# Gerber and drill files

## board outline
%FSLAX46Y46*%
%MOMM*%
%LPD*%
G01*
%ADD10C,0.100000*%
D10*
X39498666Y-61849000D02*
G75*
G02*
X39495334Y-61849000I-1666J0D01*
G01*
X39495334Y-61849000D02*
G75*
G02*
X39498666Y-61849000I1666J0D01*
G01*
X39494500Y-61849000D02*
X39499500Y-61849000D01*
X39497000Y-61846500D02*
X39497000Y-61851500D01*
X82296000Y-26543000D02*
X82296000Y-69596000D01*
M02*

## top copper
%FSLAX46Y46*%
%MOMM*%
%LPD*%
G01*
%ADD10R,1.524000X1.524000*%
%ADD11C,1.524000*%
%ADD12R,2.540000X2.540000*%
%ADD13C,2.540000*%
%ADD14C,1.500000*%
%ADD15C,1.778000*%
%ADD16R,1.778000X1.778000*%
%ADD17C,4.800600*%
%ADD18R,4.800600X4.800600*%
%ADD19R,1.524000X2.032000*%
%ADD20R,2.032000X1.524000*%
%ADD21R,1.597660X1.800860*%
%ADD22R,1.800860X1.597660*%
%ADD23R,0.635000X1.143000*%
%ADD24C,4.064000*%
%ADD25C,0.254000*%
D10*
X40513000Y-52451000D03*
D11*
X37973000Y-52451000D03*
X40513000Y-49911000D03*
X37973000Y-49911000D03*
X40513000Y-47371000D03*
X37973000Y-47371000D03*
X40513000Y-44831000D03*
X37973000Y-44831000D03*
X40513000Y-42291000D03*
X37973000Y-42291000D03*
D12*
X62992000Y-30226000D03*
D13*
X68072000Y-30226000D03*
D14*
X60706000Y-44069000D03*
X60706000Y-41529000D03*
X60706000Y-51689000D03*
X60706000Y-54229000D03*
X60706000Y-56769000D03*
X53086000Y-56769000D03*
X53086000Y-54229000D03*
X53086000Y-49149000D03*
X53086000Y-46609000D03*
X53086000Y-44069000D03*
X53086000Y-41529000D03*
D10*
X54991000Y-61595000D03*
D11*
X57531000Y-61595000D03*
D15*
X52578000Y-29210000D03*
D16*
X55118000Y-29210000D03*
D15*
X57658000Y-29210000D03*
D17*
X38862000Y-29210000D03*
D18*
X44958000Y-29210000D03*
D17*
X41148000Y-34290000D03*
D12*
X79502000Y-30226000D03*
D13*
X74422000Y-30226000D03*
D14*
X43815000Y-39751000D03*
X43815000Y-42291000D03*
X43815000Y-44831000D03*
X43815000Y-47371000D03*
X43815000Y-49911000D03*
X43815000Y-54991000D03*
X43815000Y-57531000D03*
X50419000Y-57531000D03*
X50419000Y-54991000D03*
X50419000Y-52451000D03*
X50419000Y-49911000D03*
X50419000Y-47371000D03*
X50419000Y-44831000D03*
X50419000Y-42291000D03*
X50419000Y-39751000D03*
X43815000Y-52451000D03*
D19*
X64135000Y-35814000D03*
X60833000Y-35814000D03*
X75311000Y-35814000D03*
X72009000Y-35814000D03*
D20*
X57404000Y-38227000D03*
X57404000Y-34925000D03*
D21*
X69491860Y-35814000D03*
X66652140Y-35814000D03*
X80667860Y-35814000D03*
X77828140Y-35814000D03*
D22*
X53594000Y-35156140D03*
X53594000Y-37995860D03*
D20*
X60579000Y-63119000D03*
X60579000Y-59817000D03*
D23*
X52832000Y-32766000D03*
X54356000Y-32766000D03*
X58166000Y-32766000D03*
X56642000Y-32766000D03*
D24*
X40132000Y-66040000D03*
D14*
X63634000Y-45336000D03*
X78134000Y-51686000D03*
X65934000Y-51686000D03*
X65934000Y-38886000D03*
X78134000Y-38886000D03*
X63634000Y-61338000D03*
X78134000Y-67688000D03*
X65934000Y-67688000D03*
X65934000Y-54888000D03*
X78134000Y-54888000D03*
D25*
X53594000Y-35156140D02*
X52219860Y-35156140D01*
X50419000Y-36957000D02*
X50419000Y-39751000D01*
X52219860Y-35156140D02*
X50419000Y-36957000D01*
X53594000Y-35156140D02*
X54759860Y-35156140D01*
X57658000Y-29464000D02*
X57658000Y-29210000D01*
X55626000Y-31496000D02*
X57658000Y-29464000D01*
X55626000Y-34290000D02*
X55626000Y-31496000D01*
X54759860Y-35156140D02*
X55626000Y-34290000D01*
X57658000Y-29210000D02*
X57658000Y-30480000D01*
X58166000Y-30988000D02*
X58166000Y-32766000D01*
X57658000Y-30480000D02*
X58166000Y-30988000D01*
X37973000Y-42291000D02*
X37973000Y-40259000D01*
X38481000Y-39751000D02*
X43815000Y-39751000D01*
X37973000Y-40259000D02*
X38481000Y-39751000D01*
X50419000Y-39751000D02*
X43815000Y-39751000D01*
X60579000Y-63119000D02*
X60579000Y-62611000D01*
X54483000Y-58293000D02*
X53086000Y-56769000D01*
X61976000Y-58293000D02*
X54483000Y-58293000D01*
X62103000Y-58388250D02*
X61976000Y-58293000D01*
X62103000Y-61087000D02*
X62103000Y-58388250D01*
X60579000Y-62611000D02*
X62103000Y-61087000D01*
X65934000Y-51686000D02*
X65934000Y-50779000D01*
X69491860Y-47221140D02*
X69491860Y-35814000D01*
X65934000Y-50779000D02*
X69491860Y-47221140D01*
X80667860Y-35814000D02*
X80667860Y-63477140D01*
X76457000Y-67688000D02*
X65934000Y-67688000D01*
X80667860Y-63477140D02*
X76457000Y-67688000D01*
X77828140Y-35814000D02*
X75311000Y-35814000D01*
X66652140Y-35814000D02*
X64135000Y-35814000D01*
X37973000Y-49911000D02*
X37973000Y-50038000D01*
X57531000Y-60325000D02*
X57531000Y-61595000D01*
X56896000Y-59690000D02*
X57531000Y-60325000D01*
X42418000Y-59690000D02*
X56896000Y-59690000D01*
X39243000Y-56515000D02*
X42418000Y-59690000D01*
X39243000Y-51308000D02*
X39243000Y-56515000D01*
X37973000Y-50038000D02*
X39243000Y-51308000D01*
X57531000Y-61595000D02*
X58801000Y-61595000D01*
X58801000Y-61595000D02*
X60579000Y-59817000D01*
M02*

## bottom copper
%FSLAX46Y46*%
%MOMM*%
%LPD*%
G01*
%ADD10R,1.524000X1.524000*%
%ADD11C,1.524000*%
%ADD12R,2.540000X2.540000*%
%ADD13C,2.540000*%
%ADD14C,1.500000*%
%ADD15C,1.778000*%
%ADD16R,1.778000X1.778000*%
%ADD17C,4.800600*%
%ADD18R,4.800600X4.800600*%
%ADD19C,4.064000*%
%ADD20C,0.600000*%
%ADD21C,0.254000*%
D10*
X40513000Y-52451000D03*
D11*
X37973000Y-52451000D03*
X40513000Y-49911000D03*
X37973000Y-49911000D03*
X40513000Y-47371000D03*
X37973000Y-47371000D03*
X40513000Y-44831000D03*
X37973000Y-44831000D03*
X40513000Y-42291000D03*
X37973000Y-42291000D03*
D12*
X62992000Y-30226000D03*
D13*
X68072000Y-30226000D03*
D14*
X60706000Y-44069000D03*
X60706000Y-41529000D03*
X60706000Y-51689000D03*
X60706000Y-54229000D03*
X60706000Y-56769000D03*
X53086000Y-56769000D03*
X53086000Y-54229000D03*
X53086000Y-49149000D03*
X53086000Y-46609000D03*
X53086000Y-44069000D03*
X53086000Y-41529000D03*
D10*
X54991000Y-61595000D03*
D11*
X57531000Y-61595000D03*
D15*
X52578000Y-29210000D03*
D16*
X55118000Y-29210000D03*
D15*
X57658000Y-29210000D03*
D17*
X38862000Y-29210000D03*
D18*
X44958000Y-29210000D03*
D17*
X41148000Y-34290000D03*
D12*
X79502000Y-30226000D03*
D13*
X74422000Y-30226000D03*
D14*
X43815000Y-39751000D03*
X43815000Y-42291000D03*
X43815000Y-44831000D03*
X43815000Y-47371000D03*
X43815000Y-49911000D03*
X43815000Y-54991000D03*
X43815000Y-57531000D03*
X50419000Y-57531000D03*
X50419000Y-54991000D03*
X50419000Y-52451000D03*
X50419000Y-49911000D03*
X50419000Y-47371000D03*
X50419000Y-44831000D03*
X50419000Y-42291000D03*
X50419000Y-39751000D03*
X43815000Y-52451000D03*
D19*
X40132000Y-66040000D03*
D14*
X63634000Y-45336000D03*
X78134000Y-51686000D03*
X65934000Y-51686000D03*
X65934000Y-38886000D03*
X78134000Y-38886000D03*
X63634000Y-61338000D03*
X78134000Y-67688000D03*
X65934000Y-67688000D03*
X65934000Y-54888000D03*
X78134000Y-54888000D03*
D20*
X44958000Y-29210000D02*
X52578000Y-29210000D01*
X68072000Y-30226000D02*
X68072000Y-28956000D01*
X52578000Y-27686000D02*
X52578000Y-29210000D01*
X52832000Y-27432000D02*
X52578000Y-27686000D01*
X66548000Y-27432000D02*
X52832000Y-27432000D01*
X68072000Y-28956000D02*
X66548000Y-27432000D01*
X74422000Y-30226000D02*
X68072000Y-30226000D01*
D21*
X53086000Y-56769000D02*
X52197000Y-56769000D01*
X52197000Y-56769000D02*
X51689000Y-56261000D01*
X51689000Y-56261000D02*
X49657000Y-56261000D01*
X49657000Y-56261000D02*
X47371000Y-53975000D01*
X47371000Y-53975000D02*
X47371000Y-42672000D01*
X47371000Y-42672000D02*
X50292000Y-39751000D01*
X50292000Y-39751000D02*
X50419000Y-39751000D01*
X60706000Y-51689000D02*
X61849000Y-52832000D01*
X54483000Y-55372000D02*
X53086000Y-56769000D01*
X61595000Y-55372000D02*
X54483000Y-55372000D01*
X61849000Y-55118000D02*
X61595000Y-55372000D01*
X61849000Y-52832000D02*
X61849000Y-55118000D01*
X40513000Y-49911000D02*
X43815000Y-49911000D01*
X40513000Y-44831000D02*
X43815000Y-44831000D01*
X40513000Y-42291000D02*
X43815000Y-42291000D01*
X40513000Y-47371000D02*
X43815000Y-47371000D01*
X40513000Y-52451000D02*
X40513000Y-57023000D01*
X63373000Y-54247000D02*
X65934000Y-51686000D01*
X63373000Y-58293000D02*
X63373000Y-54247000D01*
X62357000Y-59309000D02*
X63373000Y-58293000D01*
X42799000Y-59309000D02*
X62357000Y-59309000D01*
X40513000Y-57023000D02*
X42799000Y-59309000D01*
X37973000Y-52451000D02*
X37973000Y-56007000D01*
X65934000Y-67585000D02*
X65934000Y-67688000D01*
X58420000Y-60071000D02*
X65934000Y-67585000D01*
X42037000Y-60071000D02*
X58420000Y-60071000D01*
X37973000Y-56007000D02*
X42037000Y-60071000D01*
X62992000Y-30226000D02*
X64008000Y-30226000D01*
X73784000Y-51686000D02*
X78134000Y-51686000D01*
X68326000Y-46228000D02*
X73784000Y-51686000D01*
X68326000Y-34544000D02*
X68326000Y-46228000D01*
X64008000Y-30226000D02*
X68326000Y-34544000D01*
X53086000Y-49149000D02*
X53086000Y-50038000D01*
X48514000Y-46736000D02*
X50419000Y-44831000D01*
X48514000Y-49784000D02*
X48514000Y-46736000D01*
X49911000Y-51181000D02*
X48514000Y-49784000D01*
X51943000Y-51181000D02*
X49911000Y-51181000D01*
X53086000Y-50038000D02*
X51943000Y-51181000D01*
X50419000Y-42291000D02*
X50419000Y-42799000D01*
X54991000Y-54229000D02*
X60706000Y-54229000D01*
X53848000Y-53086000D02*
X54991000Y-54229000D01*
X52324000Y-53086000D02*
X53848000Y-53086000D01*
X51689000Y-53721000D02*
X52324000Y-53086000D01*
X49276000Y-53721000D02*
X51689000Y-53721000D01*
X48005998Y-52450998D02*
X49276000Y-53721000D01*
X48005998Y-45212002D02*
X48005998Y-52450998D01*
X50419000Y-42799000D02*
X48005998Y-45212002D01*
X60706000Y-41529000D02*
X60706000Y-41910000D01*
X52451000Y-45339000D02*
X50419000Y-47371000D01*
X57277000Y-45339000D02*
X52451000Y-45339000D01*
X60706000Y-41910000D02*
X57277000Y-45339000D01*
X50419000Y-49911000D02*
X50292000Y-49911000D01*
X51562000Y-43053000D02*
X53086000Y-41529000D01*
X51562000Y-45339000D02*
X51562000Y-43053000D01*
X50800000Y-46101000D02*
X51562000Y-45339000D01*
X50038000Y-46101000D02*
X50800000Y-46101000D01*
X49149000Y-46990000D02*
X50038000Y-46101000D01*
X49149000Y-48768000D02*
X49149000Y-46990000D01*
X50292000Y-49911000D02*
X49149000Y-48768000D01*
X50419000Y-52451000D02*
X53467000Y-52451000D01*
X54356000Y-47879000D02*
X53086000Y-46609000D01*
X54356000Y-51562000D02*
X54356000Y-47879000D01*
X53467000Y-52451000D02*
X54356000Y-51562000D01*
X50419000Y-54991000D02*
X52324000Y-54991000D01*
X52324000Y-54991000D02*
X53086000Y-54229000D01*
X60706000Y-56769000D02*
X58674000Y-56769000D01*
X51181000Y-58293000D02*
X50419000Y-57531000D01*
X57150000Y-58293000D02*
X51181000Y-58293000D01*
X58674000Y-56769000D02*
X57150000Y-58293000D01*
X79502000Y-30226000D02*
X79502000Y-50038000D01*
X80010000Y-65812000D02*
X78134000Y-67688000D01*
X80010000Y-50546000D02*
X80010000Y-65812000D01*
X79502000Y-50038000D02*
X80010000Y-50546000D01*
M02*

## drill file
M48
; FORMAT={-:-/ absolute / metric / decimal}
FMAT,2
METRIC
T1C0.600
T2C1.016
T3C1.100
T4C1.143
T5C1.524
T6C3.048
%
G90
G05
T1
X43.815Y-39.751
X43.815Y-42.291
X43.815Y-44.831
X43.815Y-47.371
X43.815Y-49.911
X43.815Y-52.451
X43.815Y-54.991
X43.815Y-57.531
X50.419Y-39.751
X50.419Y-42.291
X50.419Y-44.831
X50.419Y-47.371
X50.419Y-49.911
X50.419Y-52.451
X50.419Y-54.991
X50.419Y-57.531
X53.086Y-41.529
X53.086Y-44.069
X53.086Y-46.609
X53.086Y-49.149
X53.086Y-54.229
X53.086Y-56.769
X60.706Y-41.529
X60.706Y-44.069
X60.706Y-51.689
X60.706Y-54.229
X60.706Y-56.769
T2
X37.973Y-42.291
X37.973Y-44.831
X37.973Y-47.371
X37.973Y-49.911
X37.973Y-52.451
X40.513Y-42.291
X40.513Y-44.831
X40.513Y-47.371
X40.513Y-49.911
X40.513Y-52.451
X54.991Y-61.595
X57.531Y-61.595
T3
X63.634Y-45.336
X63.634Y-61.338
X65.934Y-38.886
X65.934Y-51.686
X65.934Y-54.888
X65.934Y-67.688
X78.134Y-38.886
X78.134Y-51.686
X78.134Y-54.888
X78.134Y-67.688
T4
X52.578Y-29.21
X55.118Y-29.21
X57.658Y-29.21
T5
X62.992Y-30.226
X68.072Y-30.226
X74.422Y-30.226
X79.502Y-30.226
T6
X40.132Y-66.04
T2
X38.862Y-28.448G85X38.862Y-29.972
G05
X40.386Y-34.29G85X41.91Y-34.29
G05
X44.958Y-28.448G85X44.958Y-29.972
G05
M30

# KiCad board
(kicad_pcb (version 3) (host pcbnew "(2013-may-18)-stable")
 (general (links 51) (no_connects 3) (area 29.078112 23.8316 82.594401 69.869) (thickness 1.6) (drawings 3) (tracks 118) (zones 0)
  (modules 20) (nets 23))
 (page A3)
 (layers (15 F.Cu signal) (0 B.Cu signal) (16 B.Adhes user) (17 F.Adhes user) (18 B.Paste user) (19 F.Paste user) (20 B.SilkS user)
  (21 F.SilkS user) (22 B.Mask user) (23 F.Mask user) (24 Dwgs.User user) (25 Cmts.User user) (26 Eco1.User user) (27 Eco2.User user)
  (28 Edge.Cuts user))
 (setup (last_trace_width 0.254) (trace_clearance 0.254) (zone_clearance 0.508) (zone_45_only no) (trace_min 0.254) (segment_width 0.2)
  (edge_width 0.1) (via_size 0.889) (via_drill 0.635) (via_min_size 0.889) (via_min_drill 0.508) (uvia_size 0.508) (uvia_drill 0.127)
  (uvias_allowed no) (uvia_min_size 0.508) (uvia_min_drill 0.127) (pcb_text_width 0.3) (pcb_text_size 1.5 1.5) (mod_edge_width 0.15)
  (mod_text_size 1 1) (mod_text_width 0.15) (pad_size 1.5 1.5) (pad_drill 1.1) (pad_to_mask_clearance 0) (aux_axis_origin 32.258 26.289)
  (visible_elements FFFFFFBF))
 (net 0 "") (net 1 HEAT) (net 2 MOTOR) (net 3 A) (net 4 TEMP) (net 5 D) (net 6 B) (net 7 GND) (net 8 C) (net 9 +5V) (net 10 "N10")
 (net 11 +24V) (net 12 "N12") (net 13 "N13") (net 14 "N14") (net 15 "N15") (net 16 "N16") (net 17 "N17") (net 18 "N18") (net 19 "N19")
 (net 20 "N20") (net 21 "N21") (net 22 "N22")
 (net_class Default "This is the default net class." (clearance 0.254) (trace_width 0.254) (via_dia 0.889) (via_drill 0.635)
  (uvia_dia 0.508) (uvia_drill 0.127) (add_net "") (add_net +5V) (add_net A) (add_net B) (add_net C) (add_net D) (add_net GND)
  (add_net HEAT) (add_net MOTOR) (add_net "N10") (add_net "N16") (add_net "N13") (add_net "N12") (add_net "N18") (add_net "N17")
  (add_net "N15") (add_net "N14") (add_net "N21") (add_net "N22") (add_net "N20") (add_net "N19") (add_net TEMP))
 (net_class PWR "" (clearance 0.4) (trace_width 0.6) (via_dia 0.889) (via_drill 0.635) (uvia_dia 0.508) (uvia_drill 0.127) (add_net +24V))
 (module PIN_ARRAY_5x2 (layer F.Cu) (at 39.243 47.371 90)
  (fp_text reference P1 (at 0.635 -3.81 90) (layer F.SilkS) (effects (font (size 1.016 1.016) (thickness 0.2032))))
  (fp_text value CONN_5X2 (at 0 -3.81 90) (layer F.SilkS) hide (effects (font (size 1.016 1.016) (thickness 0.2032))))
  (pad 1 thru_hole rect (at -5.08 1.27 90) (size 1.524 1.524) (drill 1.016) (layers *.Cu *.Mask F.SilkS) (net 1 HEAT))
  (pad 2 thru_hole circle (at -5.08 -1.27 90) (size 1.524 1.524) (drill 1.016) (layers *.Cu *.Mask F.SilkS) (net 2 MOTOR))
  (pad 3 thru_hole circle (at -2.54 1.27 90) (size 1.524 1.524) (drill 1.016) (layers *.Cu *.Mask F.SilkS) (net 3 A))
  (pad 4 thru_hole circle (at -2.54 -1.27 90) (size 1.524 1.524) (drill 1.016) (layers *.Cu *.Mask F.SilkS) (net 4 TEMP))
  (pad 5 thru_hole circle (at 0 1.27 90) (size 1.524 1.524) (drill 1.016) (layers *.Cu *.Mask F.SilkS) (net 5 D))
  (pad 6 thru_hole circle (at 0 -1.27 90) (size 1.524 1.524) (drill 1.016) (layers *.Cu *.Mask F.SilkS))
  (pad 7 thru_hole circle (at 2.54 1.27 90) (size 1.524 1.524) (drill 1.016) (layers *.Cu *.Mask F.SilkS) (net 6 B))
  (pad 8 thru_hole circle (at 2.54 -1.27 90) (size 1.524 1.524) (drill 1.016) (layers *.Cu *.Mask F.SilkS) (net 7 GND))
  (pad 9 thru_hole circle (at 5.08 1.27 90) (size 1.524 1.524) (drill 1.016) (layers *.Cu *.Mask F.SilkS) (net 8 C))
  (pad 10 thru_hole circle (at 5.08 -1.27 90) (size 1.524 1.524) (drill 1.016) (layers *.Cu *.Mask F.SilkS) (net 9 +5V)))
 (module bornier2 (layer F.Cu) (at 65.532 30.226)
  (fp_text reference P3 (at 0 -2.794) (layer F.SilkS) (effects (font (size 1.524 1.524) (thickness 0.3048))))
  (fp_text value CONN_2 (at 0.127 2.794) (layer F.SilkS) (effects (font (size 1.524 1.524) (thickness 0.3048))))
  (pad 1 thru_hole rect (at -2.54 0) (size 2.54 2.54) (drill 1.524) (layers *.Cu *.Mask F.SilkS) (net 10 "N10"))
  (pad 2 thru_hole circle (at 2.54 0) (size 2.54 2.54) (drill 1.524) (layers *.Cu *.Mask F.SilkS) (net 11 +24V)))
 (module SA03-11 (layer F.Cu) (at 56.896 49.149 180)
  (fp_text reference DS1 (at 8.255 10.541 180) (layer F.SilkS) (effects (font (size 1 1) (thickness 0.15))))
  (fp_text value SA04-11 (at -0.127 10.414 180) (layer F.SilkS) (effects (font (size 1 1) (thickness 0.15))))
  (pad 6 thru_hole circle (at -3.81 5.08 180) (size 1.5 1.5) (drill 0.6) (layers *.Cu *.Mask F.SilkS))
  (pad 7 thru_hole circle (at -3.81 7.62 180) (size 1.5 1.5) (drill 0.6) (layers *.Cu *.Mask F.SilkS) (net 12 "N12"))
  (pad 3 thru_hole circle (at -3.81 -2.54 180) (size 1.5 1.5) (drill 0.6) (layers *.Cu *.Mask F.SilkS) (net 9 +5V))
  (pad 2 thru_hole circle (at -3.81 -5.08 180) (size 1.5 1.5) (drill 0.6) (layers *.Cu *.Mask F.SilkS) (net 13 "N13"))
  (pad 1 thru_hole circle (at -3.81 -7.62 180) (size 1.5 1.5) (drill 0.6) (layers *.Cu *.Mask F.SilkS) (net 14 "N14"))
  (pad 14 thru_hole circle (at 3.81 -7.62 180) (size 1.5 1.5) (drill 0.6) (layers *.Cu *.Mask F.SilkS) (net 9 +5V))
  (pad 13 thru_hole circle (at 3.81 -5.08 180) (size 1.5 1.5) (drill 0.6) (layers *.Cu *.Mask F.SilkS) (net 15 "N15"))
  (pad 11 thru_hole circle (at 3.81 0 180) (size 1.5 1.5) (drill 0.6) (layers *.Cu *.Mask F.SilkS) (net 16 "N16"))
  (pad 10 thru_hole circle (at 3.81 2.54 180) (size 1.5 1.5) (drill 0.6) (layers *.Cu *.Mask F.SilkS) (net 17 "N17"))
  (pad 9 thru_hole circle (at 3.81 5.08 180) (size 1.5 1.5) (drill 0.6) (layers *.Cu *.Mask F.SilkS))
  (pad 8 thru_hole circle (at 3.81 7.62 180) (size 1.5 1.5) (drill 0.6) (layers *.Cu *.Mask F.SilkS) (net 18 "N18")))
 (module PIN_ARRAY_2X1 (layer F.Cu) (at 56.261 61.595)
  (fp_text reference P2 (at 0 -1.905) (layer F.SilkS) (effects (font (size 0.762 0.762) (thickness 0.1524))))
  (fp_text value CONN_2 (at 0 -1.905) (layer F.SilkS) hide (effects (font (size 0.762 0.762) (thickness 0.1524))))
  (pad 1 thru_hole rect (at -1.27 0) (size 1.524 1.524) (drill 1.016) (layers *.Cu *.Mask F.SilkS) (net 7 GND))
  (pad 2 thru_hole circle (at 1.27 0) (size 1.524 1.524) (drill 1.016) (layers *.Cu *.Mask F.SilkS) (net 4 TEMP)))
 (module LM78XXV (layer F.Cu) (at 55.118 29.21 90)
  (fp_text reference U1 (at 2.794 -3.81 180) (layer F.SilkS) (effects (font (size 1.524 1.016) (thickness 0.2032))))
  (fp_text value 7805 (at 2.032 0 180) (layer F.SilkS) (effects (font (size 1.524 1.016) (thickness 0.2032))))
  (pad VI thru_hole circle (at 0 -2.54 90) (size 1.778 1.778) (drill 1.143) (layers *.Cu *.Mask F.SilkS) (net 11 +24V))
  (pad GND thru_hole rect (at 0 0 90) (size 1.778 1.778) (drill 1.143) (layers *.Cu *.Mask F.SilkS) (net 7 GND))
  (pad VO thru_hole circle (at 0 2.54 90) (size 1.778 1.778) (drill 1.143) (layers *.Cu *.Mask F.SilkS) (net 9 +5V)))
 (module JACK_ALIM (layer F.Cu) (at 38.862 29.21)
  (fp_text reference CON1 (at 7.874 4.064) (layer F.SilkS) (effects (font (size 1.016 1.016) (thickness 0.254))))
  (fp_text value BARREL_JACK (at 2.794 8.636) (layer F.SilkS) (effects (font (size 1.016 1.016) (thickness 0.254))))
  (pad 2 thru_hole circle (at 0 0) (size 4.8006 4.8006) (drill oval 1.016 2.54) (layers *.Cu *.Mask F.SilkS) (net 7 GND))
  (pad 1 thru_hole rect (at 6.096 0) (size 4.8006 4.8006) (drill oval 1.016 2.54) (layers *.Cu *.Mask F.SilkS) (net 11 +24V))
  (pad 3 thru_hole circle (at 2.286 5.08) (size 4.8006 4.8006) (drill oval 2.54 1.016) (layers *.Cu *.Mask F.SilkS) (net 7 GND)))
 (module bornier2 (layer F.Cu) (at 76.962 30.226 180)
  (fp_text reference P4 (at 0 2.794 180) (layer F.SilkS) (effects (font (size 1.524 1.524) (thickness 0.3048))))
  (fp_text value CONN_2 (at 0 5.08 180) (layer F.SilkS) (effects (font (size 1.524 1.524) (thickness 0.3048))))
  (pad 1 thru_hole rect (at -2.54 0 180) (size 2.54 2.54) (drill 1.524) (layers *.Cu *.Mask F.SilkS) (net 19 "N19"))
  (pad 2 thru_hole circle (at 2.54 0 180) (size 2.54 2.54) (drill 1.524) (layers *.Cu *.Mask F.SilkS) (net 11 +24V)))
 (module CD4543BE (layer F.Cu) (at 47.117 48.641 270)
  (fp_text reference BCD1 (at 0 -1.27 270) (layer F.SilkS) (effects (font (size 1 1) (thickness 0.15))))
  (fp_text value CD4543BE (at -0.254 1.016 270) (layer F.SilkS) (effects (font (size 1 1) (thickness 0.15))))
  (pad 1 thru_hole circle (at -8.89 3.302 270) (size 1.5 1.5) (drill 0.6) (layers *.Cu *.Mask F.SilkS) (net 9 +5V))
  (pad 2 thru_hole circle (at -6.35 3.302 270) (size 1.5 1.5) (drill 0.6) (layers *.Cu *.Mask F.SilkS) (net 8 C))
  (pad 3 thru_hole circle (at -3.81 3.302 270) (size 1.5 1.5) (drill 0.6) (layers *.Cu *.Mask F.SilkS) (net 6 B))
  (pad 4 thru_hole circle (at -1.27 3.302 270) (size 1.5 1.5) (drill 0.6) (layers *.Cu *.Mask F.SilkS) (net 5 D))
  (pad 5 thru_hole circle (at 1.27 3.302 270) (size 1.5 1.5) (drill 0.6) (layers *.Cu *.Mask F.SilkS) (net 3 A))
  (pad 7 thru_hole circle (at 6.35 3.302 270) (size 1.5 1.5) (drill 0.6) (layers *.Cu *.Mask F.SilkS) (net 7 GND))
  (pad 8 thru_hole circle (at 8.89 3.302 270) (size 1.5 1.5) (drill 0.6) (layers *.Cu *.Mask F.SilkS) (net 7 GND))
  (pad 9 thru_hole circle (at 8.89 -3.302 270) (size 1.5 1.5) (drill 0.6) (layers *.Cu *.Mask F.SilkS) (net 14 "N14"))
  (pad 10 thru_hole circle (at 6.35 -3.302 270) (size 1.5 1.5) (drill 0.6) (layers *.Cu *.Mask F.SilkS) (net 15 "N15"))
  (pad 11 thru_hole circle (at 3.81 -3.302 270) (size 1.5 1.5) (drill 0.6) (layers *.Cu *.Mask F.SilkS) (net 17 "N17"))
  (pad 12 thru_hole circle (at 1.27 -3.302 270) (size 1.5 1.5) (drill 0.6) (layers *.Cu *.Mask F.SilkS) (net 18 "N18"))
  (pad 13 thru_hole circle (at -1.27 -3.302 270) (size 1.5 1.5) (drill 0.6) (layers *.Cu *.Mask F.SilkS) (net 12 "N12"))
  (pad 14 thru_hole circle (at -3.81 -3.302 270) (size 1.5 1.5) (drill 0.6) (layers *.Cu *.Mask F.SilkS) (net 16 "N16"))
  (pad 15 thru_hole circle (at -6.35 -3.302 270) (size 1.5 1.5) (drill 0.6) (layers *.Cu *.Mask F.SilkS) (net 13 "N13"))
  (pad 16 thru_hole circle (at -8.89 -3.302 270) (size 1.5 1.5) (drill 0.6) (layers *.Cu *.Mask F.SilkS) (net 9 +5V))
  (pad 6 thru_hole circle (at 3.81 3.302 270) (size 1.5 1.5) (drill 0.6) (layers *.Cu *.Mask F.SilkS)))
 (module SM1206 (layer F.Cu) (at 62.484 35.814 180)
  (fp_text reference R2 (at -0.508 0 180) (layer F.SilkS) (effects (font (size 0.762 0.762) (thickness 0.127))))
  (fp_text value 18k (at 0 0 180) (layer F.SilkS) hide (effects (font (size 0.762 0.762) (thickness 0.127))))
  (pad 1 smd rect (at -1.651 0 180) (size 1.524 2.032) (layers F.Cu F.Paste F.Mask) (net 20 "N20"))
  (pad 2 smd rect (at 1.651 0 180) (size 1.524 2.032) (layers F.Cu F.Paste F.Mask) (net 7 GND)))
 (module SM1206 (layer F.Cu) (at 73.66 35.814 180)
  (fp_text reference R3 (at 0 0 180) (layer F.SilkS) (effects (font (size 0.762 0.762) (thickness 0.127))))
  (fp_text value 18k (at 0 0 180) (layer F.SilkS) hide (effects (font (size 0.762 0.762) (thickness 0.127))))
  (pad 1 smd rect (at -1.651 0 180) (size 1.524 2.032) (layers F.Cu F.Paste F.Mask) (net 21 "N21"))
  (pad 2 smd rect (at 1.651 0 180) (size 1.524 2.032) (layers F.Cu F.Paste F.Mask) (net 7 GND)))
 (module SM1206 (layer F.Cu) (at 57.404 36.576 90)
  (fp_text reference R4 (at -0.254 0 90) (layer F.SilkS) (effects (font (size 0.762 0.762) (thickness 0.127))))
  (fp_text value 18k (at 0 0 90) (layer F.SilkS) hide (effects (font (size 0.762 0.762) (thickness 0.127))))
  (pad 1 smd rect (at -1.651 0 90) (size 1.524 2.032) (layers F.Cu F.Paste F.Mask) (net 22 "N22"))
  (pad 2 smd rect (at 1.651 0 90) (size 1.524 2.032) (layers F.Cu F.Paste F.Mask) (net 7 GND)))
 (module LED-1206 (layer F.Cu) (at 68.072 35.814 180)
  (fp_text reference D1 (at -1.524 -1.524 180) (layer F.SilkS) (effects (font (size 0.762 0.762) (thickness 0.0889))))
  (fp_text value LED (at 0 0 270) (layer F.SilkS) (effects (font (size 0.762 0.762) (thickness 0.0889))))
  (pad 1 smd rect (at -1.41986 0 180) (size 1.59766 1.80086) (layers F.Cu F.Paste F.Mask) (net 1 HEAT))
  (pad 2 smd rect (at 1.41986 0 180) (size 1.59766 1.80086) (layers F.Cu F.Paste F.Mask) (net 20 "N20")))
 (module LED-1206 (layer F.Cu) (at 79.248 35.814 180)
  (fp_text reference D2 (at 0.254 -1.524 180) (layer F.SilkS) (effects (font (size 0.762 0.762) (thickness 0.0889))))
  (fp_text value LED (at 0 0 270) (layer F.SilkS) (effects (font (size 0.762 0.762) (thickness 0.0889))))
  (pad 1 smd rect (at -1.41986 0 180) (size 1.59766 1.80086) (layers F.Cu F.Paste F.Mask) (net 2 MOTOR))
  (pad 2 smd rect (at 1.41986 0 180) (size 1.59766 1.80086) (layers F.Cu F.Paste F.Mask) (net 21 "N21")))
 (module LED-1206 (layer F.Cu) (at 53.594 36.576 270)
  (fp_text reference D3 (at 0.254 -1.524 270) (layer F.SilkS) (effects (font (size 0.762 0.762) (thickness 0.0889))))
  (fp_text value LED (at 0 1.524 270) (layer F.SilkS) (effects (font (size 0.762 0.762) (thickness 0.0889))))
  (pad 1 smd rect (at -1.41986 0 270) (size 1.59766 1.80086) (layers F.Cu F.Paste F.Mask) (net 9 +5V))
  (pad 2 smd rect (at 1.41986 0 270) (size 1.59766 1.80086) (layers F.Cu F.Paste F.Mask) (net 22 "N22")))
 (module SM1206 (layer F.Cu) (at 60.579 61.468 90)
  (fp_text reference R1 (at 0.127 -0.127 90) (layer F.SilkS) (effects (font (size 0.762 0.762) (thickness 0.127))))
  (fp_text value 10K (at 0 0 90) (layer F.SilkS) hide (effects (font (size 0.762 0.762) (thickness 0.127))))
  (pad 1 smd rect (at -1.651 0 90) (size 1.524 2.032) (layers F.Cu F.Paste F.Mask) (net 9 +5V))
  (pad 2 smd rect (at 1.651 0 90) (size 1.524 2.032) (layers F.Cu F.Paste F.Mask) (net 4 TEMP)))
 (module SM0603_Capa (layer F.Cu) (at 53.594 32.766)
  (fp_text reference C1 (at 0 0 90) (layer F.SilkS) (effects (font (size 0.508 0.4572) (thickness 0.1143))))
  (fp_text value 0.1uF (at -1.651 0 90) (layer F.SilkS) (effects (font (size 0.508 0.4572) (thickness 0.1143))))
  (pad 1 smd rect (at -0.762 0) (size 0.635 1.143) (layers F.Cu F.Paste F.Mask) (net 11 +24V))
  (pad 2 smd rect (at 0.762 0) (size 0.635 1.143) (layers F.Cu F.Paste F.Mask) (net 7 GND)))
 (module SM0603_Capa (layer F.Cu) (at 57.404 32.766 180)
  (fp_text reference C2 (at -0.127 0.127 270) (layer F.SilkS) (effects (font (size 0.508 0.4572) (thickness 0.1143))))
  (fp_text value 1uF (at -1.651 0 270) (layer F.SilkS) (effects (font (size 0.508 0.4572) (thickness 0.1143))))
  (pad 1 smd rect (at -0.762 0 180) (size 0.635 1.143) (layers F.Cu F.Paste F.Mask) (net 9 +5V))
  (pad 2 smd rect (at 0.762 0 180) (size 0.635 1.143) (layers F.Cu F.Paste F.Mask) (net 7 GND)))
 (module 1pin (layer F.Cu) (at 40.132 66.04)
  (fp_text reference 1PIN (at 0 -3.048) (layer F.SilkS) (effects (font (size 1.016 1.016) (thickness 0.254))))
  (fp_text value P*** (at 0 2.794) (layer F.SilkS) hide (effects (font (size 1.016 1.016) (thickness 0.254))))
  (pad 1 thru_hole circle (at 0 0) (size 4.064 4.064) (drill 3.048) (layers *.Cu *.Mask F.SilkS)))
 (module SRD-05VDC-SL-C (layer F.Cu) (at 81.534 53.086 180)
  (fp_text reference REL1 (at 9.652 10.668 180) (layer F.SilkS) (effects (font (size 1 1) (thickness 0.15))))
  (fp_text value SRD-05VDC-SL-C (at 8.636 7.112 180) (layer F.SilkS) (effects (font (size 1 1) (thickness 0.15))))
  (pad 5 thru_hole circle (at 17.9 7.75 180) (size 1.5 1.5) (drill 1.1) (layers *.Cu *.Mask F.SilkS) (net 7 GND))
  (pad 2 thru_hole circle (at 3.4 1.4 180) (size 1.5 1.5) (drill 1.1) (layers *.Cu *.Mask F.SilkS) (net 10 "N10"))
  (pad 1 thru_hole circle (at 15.6 1.4 180) (size 1.5 1.5) (drill 1.1) (layers *.Cu *.Mask F.SilkS) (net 1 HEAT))
  (pad 4 thru_hole circle (at 15.6 14.2 180) (size 1.5 1.5) (drill 1.1) (layers *.Cu *.Mask F.SilkS) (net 7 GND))
  (pad 3 thru_hole circle (at 3.4 14.2 180) (size 1.5 1.5) (drill 1.1) (layers *.Cu *.Mask F.SilkS) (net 7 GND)))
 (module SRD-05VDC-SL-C (layer F.Cu) (at 81.534 69.088 180)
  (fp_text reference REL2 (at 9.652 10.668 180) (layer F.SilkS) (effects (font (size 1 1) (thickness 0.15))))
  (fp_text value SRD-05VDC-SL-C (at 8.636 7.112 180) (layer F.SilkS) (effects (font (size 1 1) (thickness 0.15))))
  (pad 5 thru_hole circle (at 17.9 7.75 180) (size 1.5 1.5) (drill 1.1) (layers *.Cu *.Mask F.SilkS) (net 7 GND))
  (pad 2 thru_hole circle (at 3.4 1.4 180) (size 1.5 1.5) (drill 1.1) (layers *.Cu *.Mask F.SilkS) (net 19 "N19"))
  (pad 1 thru_hole circle (at 15.6 1.4 180) (size 1.5 1.5) (drill 1.1) (layers *.Cu *.Mask F.SilkS) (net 2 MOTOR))
  (pad 4 thru_hole circle (at 15.6 14.2 180) (size 1.5 1.5) (drill 1.1) (layers *.Cu *.Mask F.SilkS) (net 7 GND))
  (pad 3 thru_hole circle (at 3.4 14.2 180) (size 1.5 1.5) (drill 1.1) (layers *.Cu *.Mask F.SilkS) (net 7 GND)))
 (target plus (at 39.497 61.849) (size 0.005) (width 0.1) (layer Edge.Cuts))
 (gr_line (start 82.296 26.543) (end 82.296 69.596) (angle 90) (layer Edge.Cuts) (width 0.1))
 (segment (start 44.958 29.21) (end 52.578 29.21) (width 0.6) (layer B.Cu) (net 11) (status C00000))
 (segment (start 68.072 30.226) (end 68.072 28.956) (width 0.6) (layer B.Cu) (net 11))
 (segment (start 52.578 27.686) (end 52.578 29.21) (width 0.6) (layer B.Cu) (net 11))
 (segment (start 52.832 27.432) (end 52.578 27.686) (width 0.6) (layer B.Cu) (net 11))
 (segment (start 66.548 27.432) (end 52.832 27.432) (width 0.6) (layer B.Cu) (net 11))
 (segment (start 68.072 28.956) (end 66.548 27.432) (width 0.6) (layer B.Cu) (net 11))
 (segment (start 74.422 30.226) (end 68.072 30.226) (width 0.6) (layer B.Cu) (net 11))
 (segment (start 53.594 35.15614) (end 52.21986 35.15614) (width 0.254) (layer F.Cu) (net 9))
 (segment (start 50.419 36.957) (end 50.419 39.751) (width 0.254) (layer F.Cu) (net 9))
 (segment (start 52.21986 35.15614) (end 50.419 36.957) (width 0.254) (layer F.Cu) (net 9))
 (segment (start 53.594 35.15614) (end 54.75986 35.15614) (width 0.254) (layer F.Cu) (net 9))
 (segment (start 57.658 29.464) (end 57.658 29.21) (width 0.254) (layer F.Cu) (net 9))
 (segment (start 55.626 31.496) (end 57.658 29.464) (width 0.254) (layer F.Cu) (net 9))
 (segment (start 55.626 34.29) (end 55.626 31.496) (width 0.254) (layer F.Cu) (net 9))
 (segment (start 54.75986 35.15614) (end 55.626 34.29) (width 0.254) (layer F.Cu) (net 9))
 (segment (start 57.658 29.21) (end 57.658 30.48) (width 0.254) (layer F.Cu) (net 9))
 (segment (start 58.166 30.988) (end 58.166 32.766) (width 0.254) (layer F.Cu) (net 9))
 (segment (start 57.658 30.48) (end 58.166 30.988) (width 0.254) (layer F.Cu) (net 9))
 (segment (start 37.973 42.291) (end 37.973 40.259) (width 0.254) (layer F.Cu) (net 9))
 (segment (start 38.481 39.751) (end 43.815 39.751) (width 0.254) (layer F.Cu) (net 9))
 (segment (start 37.973 40.259) (end 38.481 39.751) (width 0.254) (layer F.Cu) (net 9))
 (segment (start 50.419 39.751) (end 43.815 39.751) (width 0.254) (layer F.Cu) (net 9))
 (segment (start 60.579 63.119) (end 60.579 62.611) (width 0.254) (layer F.Cu) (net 9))
 (segment (start 54.483 58.293) (end 53.086 56.769) (width 0.254) (layer F.Cu) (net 9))
 (segment (start 61.976 58.293) (end 54.483 58.293) (width 0.254) (layer F.Cu) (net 9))
 (segment (start 62.103 58.38825) (end 61.976 58.293) (width 0.254) (layer F.Cu) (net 9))
 (segment (start 62.103 61.087) (end 62.103 58.38825) (width 0.254) (layer F.Cu) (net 9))
 (segment (start 60.579 62.611) (end 62.103 61.087) (width 0.254) (layer F.Cu) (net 9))
 (segment (start 53.086 56.769) (end 52.197 56.769) (width 0.254) (layer B.Cu) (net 9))
 (segment (start 52.197 56.769) (end 51.689 56.261) (width 0.254) (layer B.Cu) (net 9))
 (segment (start 51.689 56.261) (end 49.657 56.261) (width 0.254) (layer B.Cu) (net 9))
 (segment (start 49.657 56.261) (end 47.371 53.975) (width 0.254) (layer B.Cu) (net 9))
 (segment (start 47.371 53.975) (end 47.371 42.672) (width 0.254) (layer B.Cu) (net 9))
 (segment (start 47.371 42.672) (end 50.292 39.751) (width 0.254) (layer B.Cu) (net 9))
 (segment (start 50.292 39.751) (end 50.419 39.751) (width 0.254) (layer B.Cu) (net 9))
 (segment (start 60.706 51.689) (end 61.849 52.832) (width 0.254) (layer B.Cu) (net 9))
 (segment (start 54.483 55.372) (end 53.086 56.769) (width 0.254) (layer B.Cu) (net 9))
 (segment (start 61.595 55.372) (end 54.483 55.372) (width 0.254) (layer B.Cu) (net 9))
 (segment (start 61.849 55.118) (end 61.595 55.372) (width 0.254) (layer B.Cu) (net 9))
 (segment (start 61.849 52.832) (end 61.849 55.118) (width 0.254) (layer B.Cu) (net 9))
 (segment (start 40.513 49.911) (end 43.815 49.911) (width 0.254) (layer B.Cu) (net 3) (status 10))
 (segment (start 40.513 44.831) (end 43.815 44.831) (width 0.254) (layer B.Cu) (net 6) (status 10))
 (segment (start 40.513 42.291) (end 43.815 42.291) (width 0.254) (layer B.Cu) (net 8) (status 10))
 (segment (start 40.513 47.371) (end 43.815 47.371) (width 0.254) (layer B.Cu) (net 5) (status 10))
 (segment (start 40.513 52.451) (end 40.513 57.023) (width 0.254) (layer B.Cu) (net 1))
 (segment (start 63.373 54.247) (end 65.934 51.686) (width 0.254) (layer B.Cu) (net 1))
 (segment (start 63.373 58.293) (end 63.373 54.247) (width 0.254) (layer B.Cu) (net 1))
 (segment (start 62.357 59.309) (end 63.373 58.293) (width 0.254) (layer B.Cu) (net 1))
 (segment (start 42.799 59.309) (end 62.357 59.309) (width 0.254) (layer B.Cu) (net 1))
 (segment (start 40.513 57.023) (end 42.799 59.309) (width 0.254) (layer B.Cu) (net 1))
 (segment (start 65.934 51.686) (end 65.934 50.779) (width 0.254) (layer F.Cu) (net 1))
 (segment (start 69.49186 47.22114) (end 69.49186 35.814) (width 0.254) (layer F.Cu) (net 1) (status 20))
 (segment (start 65.934 50.779) (end 69.49186 47.22114) (width 0.254) (layer F.Cu) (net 1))
 (segment (start 37.973 52.451) (end 37.973 56.007) (width 0.254) (layer B.Cu) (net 2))
 (segment (start 65.934 67.585) (end 65.934 67.688) (width 0.254) (layer B.Cu) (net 2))
 (segment (start 58.42 60.071) (end 65.934 67.585) (width 0.254) (layer B.Cu) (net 2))
 (segment (start 42.037 60.071) (end 58.42 60.071) (width 0.254) (layer B.Cu) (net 2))
 (segment (start 37.973 56.007) (end 42.037 60.071) (width 0.254) (layer B.Cu) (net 2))
 (segment (start 80.66786 35.814) (end 80.66786 63.47714) (width 0.254) (layer F.Cu) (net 2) (status 10))
 (segment (start 76.457 67.688) (end 65.934 67.688) (width 0.254) (layer F.Cu) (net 2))
 (segment (start 80.66786 63.47714) (end 76.457 67.688) (width 0.254) (layer F.Cu) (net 2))
 (segment (start 62.992 30.226) (end 64.008 30.226) (width 0.254) (layer B.Cu) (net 10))
 (segment (start 73.784 51.686) (end 78.134 51.686) (width 0.254) (layer B.Cu) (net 10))
 (segment (start 68.326 46.228) (end 73.784 51.686) (width 0.254) (layer B.Cu) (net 10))
 (segment (start 68.326 34.544) (end 68.326 46.228) (width 0.254) (layer B.Cu) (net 10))
 (segment (start 64.008 30.226) (end 68.326 34.544) (width 0.254) (layer B.Cu) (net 10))
 (segment (start 53.086 49.149) (end 53.086 50.038) (width 0.254) (layer B.Cu) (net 16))
 (segment (start 48.514 46.736) (end 50.419 44.831) (width 0.254) (layer B.Cu) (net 16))
 (segment (start 48.514 49.784) (end 48.514 46.736) (width 0.254) (layer B.Cu) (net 16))
 (segment (start 49.911 51.181) (end 48.514 49.784) (width 0.254) (layer B.Cu) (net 16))
 (segment (start 51.943 51.181) (end 49.911 51.181) (width 0.254) (layer B.Cu) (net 16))
 (segment (start 53.086 50.038) (end 51.943 51.181) (width 0.254) (layer B.Cu) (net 16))
 (segment (start 50.419 42.291) (end 50.419 42.799) (width 0.254) (layer B.Cu) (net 13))
 (segment (start 54.991 54.229) (end 60.706 54.229) (width 0.254) (layer B.Cu) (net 13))
 (segment (start 53.848 53.086) (end 54.991 54.229) (width 0.254) (layer B.Cu) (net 13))
 (segment (start 52.324 53.086) (end 53.848 53.086) (width 0.254) (layer B.Cu) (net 13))
 (segment (start 51.689 53.721) (end 52.324 53.086) (width 0.254) (layer B.Cu) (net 13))
 (segment (start 49.276 53.721) (end 51.689 53.721) (width 0.254) (layer B.Cu) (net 13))
 (segment (start 48.005998 52.450998) (end 49.276 53.721) (width 0.254) (layer B.Cu) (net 13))
 (segment (start 48.005998 45.212002) (end 48.005998 52.450998) (width 0.254) (layer B.Cu) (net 13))
 (segment (start 50.419 42.799) (end 48.005998 45.212002) (width 0.254) (layer B.Cu) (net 13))
 (segment (start 60.706 41.529) (end 60.706 41.91) (width 0.254) (layer B.Cu) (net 12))
 (segment (start 52.451 45.339) (end 50.419 47.371) (width 0.254) (layer B.Cu) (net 12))
 (segment (start 57.277 45.339) (end 52.451 45.339) (width 0.254) (layer B.Cu) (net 12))
 (segment (start 60.706 41.91) (end 57.277 45.339) (width 0.254) (layer B.Cu) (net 12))
 (segment (start 50.419 49.911) (end 50.292 49.911) (width 0.254) (layer B.Cu) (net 18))
 (segment (start 51.562 43.053) (end 53.086 41.529) (width 0.254) (layer B.Cu) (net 18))
 (segment (start 51.562 45.339) (end 51.562 43.053) (width 0.254) (layer B.Cu) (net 18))
 (segment (start 50.8 46.101) (end 51.562 45.339) (width 0.254) (layer B.Cu) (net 18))
 (segment (start 50.038 46.101) (end 50.8 46.101) (width 0.254) (layer B.Cu) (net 18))
 (segment (start 49.149 46.99) (end 50.038 46.101) (width 0.254) (layer B.Cu) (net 18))
 (segment (start 49.149 48.768) (end 49.149 46.99) (width 0.254) (layer B.Cu) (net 18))
 (segment (start 50.292 49.911) (end 49.149 48.768) (width 0.254) (layer B.Cu) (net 18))
 (segment (start 50.419 52.451) (end 53.467 52.451) (width 0.254) (layer B.Cu) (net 17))
 (segment (start 54.356 47.879) (end 53.086 46.609) (width 0.254) (layer B.Cu) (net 17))
 (segment (start 54.356 51.562) (end 54.356 47.879) (width 0.254) (layer B.Cu) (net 17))
 (segment (start 53.467 52.451) (end 54.356 51.562) (width 0.254) (layer B.Cu) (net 17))
 (segment (start 50.419 54.991) (end 52.324 54.991) (width 0.254) (layer B.Cu) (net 15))
 (segment (start 52.324 54.991) (end 53.086 54.229) (width 0.254) (layer B.Cu) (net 15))
 (segment (start 60.706 56.769) (end 58.674 56.769) (width 0.254) (layer B.Cu) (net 14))
 (segment (start 51.181 58.293) (end 50.419 57.531) (width 0.254) (layer B.Cu) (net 14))
 (segment (start 57.15 58.293) (end 51.181 58.293) (width 0.254) (layer B.Cu) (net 14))
 (segment (start 58.674 56.769) (end 57.15 58.293) (width 0.254) (layer B.Cu) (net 14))
 (segment (start 77.82814 35.814) (end 75.311 35.814) (width 0.254) (layer F.Cu) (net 21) (status 20))
 (segment (start 66.65214 35.814) (end 64.135 35.814) (width 0.254) (layer F.Cu) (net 20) (status 20))
 (segment (start 79.502 30.226) (end 79.502 50.038) (width 0.254) (layer B.Cu) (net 19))
 (segment (start 80.01 65.812) (end 78.134 67.688) (width 0.254) (layer B.Cu) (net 19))
 (segment (start 80.01 50.546) (end 80.01 65.812) (width 0.254) (layer B.Cu) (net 19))
 (segment (start 79.502 50.038) (end 80.01 50.546) (width 0.254) (layer B.Cu) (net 19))
 (segment (start 37.973 49.911) (end 37.973 50.038) (width 0.254) (layer F.Cu) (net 4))
 (segment (start 57.531 60.325) (end 57.531 61.595) (width 0.254) (layer F.Cu) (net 4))
 (segment (start 56.896 59.69) (end 57.531 60.325) (width 0.254) (layer F.Cu) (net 4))
 (segment (start 42.418 59.69) (end 56.896 59.69) (width 0.254) (layer F.Cu) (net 4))
 (segment (start 39.243 56.515) (end 42.418 59.69) (width 0.254) (layer F.Cu) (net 4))
 (segment (start 39.243 51.308) (end 39.243 56.515) (width 0.254) (layer F.Cu) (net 4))
 (segment (start 37.973 50.038) (end 39.243 51.308) (width 0.254) (layer F.Cu) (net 4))
 (segment (start 57.531 61.595) (end 58.801 61.595) (width 0.254) (layer F.Cu) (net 4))
 (segment (start 58.801 61.595) (end 60.579 59.817) (width 0.254) (layer F.Cu) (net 4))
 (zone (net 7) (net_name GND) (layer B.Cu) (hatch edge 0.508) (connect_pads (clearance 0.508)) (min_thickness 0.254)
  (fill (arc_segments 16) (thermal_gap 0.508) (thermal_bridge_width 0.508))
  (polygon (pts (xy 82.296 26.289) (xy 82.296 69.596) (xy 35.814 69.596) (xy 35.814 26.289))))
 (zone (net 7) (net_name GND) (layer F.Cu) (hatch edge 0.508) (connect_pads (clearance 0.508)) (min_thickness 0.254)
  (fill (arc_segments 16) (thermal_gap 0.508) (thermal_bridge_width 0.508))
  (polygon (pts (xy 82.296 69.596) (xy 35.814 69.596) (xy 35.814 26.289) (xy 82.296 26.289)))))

